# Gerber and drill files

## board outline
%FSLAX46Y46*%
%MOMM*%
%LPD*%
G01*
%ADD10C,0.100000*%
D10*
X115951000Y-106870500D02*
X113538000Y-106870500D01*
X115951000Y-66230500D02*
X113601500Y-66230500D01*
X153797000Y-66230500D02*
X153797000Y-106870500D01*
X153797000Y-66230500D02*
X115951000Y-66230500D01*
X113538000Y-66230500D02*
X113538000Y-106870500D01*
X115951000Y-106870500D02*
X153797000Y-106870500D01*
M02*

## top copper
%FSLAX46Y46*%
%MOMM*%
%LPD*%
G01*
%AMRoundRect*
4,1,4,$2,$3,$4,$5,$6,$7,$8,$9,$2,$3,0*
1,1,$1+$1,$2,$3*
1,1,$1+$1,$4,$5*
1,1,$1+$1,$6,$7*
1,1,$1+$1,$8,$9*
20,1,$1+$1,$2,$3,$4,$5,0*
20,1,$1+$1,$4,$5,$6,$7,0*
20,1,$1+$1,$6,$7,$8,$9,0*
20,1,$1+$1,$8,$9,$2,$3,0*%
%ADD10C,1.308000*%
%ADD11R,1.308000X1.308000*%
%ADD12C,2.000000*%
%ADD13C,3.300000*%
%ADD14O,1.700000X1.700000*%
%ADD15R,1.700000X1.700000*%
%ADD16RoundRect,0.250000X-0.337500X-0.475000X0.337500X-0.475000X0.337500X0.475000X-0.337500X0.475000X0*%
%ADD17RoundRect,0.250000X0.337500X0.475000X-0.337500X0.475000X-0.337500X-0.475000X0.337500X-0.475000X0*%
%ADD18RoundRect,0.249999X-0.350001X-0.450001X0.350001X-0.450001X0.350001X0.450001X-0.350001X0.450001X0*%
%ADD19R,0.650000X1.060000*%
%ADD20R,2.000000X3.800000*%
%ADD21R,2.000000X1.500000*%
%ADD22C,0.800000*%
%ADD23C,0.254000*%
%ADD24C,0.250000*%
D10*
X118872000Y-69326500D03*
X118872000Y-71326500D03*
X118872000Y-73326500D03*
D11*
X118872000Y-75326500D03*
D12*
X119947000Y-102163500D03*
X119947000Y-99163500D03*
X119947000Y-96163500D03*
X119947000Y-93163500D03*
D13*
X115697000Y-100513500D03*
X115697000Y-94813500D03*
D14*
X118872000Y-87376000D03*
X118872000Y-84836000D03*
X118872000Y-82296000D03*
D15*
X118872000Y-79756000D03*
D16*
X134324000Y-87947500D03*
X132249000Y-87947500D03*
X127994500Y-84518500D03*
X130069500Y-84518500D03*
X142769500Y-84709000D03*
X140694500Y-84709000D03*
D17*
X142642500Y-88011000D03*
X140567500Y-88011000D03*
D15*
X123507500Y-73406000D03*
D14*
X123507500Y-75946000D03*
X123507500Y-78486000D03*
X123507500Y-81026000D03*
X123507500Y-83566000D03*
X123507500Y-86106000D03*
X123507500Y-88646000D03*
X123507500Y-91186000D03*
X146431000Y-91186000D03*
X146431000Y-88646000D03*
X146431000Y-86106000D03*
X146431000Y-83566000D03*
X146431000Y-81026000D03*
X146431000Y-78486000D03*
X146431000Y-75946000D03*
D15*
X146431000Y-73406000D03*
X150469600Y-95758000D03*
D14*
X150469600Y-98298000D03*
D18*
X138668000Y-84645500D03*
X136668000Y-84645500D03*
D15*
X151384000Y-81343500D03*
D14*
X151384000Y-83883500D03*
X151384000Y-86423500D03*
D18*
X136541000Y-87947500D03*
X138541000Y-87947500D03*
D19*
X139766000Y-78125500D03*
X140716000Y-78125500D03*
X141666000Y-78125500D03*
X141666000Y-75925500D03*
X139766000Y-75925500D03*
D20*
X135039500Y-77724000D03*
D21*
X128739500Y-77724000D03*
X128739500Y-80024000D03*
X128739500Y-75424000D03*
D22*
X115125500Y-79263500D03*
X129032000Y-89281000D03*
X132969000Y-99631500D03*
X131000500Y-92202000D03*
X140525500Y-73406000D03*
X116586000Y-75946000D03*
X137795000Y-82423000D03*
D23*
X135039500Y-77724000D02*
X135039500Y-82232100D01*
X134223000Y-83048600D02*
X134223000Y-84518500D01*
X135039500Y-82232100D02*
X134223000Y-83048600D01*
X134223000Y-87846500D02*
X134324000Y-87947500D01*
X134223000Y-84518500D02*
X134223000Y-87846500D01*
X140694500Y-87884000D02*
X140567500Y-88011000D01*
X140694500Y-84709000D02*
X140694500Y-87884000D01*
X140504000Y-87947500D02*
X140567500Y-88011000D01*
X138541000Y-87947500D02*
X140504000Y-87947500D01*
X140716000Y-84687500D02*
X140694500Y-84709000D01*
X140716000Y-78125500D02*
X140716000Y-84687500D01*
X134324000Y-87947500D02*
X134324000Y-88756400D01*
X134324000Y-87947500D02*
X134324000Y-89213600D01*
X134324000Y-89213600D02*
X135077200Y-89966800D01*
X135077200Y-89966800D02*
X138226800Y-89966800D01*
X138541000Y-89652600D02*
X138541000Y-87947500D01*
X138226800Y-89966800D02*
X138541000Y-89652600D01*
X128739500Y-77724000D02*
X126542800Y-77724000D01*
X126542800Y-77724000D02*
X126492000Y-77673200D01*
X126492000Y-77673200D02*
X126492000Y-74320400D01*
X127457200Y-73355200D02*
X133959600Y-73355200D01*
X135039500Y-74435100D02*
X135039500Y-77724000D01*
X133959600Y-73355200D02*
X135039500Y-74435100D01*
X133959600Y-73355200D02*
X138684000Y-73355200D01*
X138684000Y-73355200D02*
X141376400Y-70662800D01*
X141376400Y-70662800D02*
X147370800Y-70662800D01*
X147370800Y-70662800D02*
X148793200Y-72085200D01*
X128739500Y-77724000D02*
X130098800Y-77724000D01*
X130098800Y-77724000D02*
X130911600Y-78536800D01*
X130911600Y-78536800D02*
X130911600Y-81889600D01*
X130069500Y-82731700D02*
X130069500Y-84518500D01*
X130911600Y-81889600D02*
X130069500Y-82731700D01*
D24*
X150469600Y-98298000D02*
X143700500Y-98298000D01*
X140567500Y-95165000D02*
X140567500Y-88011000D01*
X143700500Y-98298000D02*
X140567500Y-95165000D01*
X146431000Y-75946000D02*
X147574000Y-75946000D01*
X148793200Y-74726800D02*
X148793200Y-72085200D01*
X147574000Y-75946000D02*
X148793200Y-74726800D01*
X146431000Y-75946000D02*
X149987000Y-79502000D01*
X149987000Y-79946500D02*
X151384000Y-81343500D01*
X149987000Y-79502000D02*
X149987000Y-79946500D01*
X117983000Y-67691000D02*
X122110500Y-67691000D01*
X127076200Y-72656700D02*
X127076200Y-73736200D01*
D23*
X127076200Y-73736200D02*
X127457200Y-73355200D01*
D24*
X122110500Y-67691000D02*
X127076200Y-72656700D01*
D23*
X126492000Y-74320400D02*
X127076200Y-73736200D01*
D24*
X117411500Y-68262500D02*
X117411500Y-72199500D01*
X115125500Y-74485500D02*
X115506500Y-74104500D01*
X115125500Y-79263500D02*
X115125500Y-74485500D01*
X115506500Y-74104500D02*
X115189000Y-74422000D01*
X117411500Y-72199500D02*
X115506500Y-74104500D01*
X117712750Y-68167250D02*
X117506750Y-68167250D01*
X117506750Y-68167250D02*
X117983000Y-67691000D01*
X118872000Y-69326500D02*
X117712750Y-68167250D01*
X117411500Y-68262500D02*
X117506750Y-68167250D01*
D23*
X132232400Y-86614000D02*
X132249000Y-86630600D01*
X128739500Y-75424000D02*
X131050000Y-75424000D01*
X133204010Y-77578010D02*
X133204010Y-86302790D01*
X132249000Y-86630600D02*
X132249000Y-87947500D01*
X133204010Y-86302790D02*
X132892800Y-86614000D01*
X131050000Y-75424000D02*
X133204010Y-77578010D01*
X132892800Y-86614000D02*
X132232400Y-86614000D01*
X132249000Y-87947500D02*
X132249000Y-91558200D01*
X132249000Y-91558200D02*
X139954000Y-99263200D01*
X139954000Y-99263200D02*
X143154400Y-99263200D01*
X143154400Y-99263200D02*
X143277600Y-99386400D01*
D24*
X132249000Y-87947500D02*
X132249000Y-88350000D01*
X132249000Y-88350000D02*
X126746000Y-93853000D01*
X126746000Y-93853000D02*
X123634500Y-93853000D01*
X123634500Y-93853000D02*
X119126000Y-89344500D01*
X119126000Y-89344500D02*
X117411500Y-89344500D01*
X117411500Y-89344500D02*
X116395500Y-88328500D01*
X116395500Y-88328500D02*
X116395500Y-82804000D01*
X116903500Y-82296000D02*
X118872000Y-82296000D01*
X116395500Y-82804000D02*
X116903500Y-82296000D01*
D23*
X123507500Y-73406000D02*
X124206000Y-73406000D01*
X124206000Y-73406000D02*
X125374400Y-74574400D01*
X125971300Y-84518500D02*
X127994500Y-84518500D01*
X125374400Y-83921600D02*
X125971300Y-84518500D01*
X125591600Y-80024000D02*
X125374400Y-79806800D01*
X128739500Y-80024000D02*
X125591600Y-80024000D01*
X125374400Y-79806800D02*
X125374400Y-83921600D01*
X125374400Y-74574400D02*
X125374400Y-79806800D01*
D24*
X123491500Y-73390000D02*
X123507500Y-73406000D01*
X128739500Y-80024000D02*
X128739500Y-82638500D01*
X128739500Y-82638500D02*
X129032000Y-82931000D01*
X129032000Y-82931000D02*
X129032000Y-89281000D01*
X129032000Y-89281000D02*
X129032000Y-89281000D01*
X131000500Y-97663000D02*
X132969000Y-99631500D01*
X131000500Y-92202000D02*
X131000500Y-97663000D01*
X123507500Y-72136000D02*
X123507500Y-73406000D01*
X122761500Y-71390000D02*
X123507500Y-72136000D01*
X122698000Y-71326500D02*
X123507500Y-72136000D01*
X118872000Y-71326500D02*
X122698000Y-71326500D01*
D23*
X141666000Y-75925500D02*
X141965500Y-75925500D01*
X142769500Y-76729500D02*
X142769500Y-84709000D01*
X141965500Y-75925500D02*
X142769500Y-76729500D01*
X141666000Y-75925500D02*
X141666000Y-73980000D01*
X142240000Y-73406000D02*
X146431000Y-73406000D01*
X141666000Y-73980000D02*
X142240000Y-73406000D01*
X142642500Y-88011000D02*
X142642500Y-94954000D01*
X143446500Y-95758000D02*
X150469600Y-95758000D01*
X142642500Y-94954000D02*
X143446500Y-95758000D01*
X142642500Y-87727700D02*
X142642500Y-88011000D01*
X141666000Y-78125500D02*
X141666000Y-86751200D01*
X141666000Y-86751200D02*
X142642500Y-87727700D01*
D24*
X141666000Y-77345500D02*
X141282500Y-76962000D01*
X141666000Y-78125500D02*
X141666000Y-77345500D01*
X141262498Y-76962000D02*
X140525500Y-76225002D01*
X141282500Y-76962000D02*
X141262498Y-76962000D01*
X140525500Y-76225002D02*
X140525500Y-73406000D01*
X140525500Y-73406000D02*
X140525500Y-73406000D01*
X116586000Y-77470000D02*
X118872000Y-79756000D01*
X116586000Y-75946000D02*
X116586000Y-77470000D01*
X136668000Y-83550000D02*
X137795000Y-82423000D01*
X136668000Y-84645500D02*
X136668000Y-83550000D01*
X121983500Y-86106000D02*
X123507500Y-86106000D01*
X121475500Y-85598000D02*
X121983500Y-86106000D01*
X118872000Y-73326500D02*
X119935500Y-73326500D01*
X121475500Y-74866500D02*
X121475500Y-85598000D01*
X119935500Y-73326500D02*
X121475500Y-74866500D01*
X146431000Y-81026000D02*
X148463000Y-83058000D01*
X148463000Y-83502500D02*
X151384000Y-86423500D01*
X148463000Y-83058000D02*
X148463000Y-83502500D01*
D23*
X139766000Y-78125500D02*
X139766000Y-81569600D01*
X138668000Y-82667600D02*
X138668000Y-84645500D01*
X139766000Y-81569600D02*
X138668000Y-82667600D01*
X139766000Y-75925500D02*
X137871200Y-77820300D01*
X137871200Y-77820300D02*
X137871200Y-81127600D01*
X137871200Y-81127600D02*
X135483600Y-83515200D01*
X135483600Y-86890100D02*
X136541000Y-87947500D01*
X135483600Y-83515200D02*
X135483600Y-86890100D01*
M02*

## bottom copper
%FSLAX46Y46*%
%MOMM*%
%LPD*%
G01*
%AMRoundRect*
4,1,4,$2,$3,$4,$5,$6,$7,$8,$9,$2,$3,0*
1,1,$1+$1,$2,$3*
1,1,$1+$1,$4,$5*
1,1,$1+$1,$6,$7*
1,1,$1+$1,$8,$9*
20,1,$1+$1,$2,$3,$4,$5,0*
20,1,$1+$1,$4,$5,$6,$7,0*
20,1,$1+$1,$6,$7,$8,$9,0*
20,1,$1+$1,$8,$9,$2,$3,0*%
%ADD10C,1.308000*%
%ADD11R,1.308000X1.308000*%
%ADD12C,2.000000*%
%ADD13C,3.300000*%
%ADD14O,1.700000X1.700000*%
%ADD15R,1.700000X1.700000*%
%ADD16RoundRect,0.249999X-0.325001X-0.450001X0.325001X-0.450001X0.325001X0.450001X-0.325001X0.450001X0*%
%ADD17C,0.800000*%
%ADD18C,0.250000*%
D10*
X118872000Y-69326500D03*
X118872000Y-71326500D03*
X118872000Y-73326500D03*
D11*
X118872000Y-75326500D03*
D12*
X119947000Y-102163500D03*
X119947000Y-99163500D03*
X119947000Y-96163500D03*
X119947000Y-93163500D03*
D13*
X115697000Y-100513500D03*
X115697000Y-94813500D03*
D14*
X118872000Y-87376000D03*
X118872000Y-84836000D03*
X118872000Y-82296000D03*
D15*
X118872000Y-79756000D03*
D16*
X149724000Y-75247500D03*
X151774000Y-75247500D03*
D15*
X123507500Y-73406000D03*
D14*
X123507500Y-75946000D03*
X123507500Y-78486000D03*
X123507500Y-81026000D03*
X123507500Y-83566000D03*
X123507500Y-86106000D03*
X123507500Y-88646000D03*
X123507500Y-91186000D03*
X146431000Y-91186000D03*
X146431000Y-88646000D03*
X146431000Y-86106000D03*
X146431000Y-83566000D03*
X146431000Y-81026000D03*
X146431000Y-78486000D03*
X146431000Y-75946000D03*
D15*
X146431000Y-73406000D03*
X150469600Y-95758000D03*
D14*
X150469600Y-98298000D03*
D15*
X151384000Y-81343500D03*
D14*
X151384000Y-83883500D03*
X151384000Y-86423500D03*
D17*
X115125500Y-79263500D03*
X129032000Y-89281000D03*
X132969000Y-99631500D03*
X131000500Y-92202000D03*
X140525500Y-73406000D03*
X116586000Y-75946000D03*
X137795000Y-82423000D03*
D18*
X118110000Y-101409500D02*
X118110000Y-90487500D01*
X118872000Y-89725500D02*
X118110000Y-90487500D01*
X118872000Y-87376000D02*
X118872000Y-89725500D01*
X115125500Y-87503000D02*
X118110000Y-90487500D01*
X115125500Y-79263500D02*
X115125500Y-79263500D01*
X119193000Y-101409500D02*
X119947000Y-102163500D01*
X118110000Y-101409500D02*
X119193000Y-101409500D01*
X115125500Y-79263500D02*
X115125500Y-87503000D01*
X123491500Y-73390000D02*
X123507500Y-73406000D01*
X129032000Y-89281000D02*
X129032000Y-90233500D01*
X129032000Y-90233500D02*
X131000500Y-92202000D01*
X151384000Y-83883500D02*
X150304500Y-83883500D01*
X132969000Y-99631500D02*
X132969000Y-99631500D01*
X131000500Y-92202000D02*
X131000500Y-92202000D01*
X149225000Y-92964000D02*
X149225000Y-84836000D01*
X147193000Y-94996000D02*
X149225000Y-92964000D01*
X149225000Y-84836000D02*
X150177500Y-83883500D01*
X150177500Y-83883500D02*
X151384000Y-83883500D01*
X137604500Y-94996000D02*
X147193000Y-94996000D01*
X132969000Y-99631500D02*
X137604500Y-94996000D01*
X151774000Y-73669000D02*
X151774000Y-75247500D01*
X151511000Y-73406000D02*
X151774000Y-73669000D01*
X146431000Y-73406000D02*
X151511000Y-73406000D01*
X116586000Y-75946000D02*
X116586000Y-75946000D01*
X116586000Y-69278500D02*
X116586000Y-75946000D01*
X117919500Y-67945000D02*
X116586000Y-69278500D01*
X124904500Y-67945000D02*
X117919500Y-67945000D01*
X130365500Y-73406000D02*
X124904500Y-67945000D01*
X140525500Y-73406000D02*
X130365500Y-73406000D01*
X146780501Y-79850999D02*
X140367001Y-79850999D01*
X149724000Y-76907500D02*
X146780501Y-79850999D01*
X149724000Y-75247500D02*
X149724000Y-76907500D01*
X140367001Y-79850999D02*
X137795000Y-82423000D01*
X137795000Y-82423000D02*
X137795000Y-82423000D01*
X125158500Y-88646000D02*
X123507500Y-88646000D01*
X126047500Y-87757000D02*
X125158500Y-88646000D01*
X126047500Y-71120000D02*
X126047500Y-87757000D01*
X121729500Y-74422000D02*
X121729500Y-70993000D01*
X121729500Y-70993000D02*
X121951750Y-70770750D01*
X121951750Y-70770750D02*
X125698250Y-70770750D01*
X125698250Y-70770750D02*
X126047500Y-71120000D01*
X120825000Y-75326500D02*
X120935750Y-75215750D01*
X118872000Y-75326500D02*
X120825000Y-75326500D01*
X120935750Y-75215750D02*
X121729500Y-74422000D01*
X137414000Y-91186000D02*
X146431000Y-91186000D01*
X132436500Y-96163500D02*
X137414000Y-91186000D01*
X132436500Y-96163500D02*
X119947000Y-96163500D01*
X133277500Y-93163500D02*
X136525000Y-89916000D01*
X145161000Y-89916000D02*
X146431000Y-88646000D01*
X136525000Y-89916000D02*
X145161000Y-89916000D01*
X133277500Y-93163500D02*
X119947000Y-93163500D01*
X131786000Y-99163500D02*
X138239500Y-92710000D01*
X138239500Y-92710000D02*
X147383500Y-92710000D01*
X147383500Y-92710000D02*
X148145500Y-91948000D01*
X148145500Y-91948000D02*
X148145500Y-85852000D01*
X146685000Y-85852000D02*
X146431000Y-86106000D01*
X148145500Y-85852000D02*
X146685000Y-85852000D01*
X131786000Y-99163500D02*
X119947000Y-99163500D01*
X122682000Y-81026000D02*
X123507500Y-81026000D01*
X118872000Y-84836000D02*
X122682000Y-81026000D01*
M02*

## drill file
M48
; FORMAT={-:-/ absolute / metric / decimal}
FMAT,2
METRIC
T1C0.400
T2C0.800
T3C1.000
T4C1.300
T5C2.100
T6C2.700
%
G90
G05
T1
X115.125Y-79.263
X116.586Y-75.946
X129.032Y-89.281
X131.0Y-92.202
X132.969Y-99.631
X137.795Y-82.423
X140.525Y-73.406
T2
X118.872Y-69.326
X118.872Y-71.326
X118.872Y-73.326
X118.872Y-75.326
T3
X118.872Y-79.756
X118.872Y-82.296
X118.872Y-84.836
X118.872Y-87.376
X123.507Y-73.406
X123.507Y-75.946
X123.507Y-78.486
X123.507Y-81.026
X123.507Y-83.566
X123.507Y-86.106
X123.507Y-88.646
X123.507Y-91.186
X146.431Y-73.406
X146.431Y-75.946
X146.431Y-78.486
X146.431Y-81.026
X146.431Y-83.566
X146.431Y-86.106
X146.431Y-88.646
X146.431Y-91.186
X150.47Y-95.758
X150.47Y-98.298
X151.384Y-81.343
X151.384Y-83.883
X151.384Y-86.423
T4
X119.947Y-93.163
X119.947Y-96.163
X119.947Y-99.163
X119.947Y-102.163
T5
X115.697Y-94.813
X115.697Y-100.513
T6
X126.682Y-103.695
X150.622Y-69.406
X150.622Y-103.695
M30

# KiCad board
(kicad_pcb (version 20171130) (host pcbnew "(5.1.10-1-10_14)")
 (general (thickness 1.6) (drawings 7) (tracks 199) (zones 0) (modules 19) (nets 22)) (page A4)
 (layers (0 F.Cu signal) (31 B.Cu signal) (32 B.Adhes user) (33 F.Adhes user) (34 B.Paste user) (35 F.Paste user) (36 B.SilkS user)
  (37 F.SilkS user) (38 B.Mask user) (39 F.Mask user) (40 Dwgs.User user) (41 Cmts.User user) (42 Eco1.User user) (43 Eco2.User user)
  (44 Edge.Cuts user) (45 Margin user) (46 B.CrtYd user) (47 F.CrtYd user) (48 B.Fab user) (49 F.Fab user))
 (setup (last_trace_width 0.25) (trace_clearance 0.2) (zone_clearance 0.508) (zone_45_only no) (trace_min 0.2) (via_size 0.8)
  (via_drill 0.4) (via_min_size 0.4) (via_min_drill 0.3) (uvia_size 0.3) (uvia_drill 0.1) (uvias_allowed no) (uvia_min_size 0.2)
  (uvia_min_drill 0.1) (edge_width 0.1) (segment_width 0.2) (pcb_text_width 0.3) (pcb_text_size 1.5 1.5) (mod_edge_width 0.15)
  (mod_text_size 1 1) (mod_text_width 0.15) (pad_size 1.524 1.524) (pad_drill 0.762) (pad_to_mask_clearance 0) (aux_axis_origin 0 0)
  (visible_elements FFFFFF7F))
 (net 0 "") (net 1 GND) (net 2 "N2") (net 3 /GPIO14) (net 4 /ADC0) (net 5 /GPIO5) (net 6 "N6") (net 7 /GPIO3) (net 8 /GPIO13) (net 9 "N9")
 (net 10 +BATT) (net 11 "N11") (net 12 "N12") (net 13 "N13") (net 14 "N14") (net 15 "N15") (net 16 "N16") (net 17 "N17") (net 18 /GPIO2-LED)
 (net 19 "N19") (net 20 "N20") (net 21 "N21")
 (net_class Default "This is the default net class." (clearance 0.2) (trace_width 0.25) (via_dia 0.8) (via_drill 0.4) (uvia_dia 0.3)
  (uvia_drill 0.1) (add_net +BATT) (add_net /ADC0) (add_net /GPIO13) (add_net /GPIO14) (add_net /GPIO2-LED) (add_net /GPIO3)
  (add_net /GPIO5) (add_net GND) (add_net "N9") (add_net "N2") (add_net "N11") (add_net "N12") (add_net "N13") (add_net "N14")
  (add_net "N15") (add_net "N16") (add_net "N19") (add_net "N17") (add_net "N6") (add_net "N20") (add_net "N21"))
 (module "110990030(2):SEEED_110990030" (layer F.Cu) (at 118.872 72.3265 90)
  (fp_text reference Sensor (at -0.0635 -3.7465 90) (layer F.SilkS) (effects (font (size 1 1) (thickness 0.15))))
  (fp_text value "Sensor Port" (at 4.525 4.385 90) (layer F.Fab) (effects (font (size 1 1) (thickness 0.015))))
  (pad 4 thru_hole circle (at 3 0 90) (size 1.308 1.308) (drill 0.8) (layers *.Cu *.Mask) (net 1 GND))
  (pad 3 thru_hole circle (at 1 0 90) (size 1.308 1.308) (drill 0.8) (layers *.Cu *.Mask) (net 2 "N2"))
  (pad 2 thru_hole circle (at -1 0 90) (size 1.308 1.308) (drill 0.8) (layers *.Cu *.Mask) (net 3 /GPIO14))
  (pad 1 thru_hole rect (at -3 0 90) (size 1.308 1.308) (drill 0.8) (layers *.Cu *.Mask) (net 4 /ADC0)))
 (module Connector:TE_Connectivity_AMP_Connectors (layer F.Cu) (at 115.697 95.3135 270)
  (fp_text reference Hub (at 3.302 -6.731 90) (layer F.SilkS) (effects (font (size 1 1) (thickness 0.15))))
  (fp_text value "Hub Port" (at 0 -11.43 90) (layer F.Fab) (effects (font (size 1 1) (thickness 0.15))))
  (pad 4 thru_hole circle (at 6.85 -4.25 270) (size 2 2) (drill 1.3) (layers *.Cu *.Mask) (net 1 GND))
  (pad 3 thru_hole circle (at 3.85 -4.25 270) (size 2 2) (drill 1.3) (layers *.Cu *.Mask) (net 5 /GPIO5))
  (pad 2 thru_hole circle (at 0.85 -4.25 270) (size 2 2) (drill 1.3) (layers *.Cu *.Mask) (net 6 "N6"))
  (pad 1 thru_hole circle (at -2.15 -4.25 270) (size 2 2) (drill 1.3) (layers *.Cu *.Mask) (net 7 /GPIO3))
  (pad 6 thru_hole circle (at 5.2 0 270) (size 3.3 3.3) (drill 2.1) (layers *.Cu *.Mask))
  (pad 5 thru_hole circle (at -0.5 0 270) (size 3.3 3.3) (drill 2.1) (layers *.Cu *.Mask)))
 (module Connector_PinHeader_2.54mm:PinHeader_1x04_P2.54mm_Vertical (layer F.Cu) (at 118.872 79.756)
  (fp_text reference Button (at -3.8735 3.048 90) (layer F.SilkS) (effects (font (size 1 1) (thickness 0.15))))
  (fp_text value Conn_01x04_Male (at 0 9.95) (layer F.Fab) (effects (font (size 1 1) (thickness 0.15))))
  (pad 4 thru_hole oval (at 0 7.62) (size 1.7 1.7) (drill 1) (layers *.Cu *.Mask) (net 1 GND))
  (pad 3 thru_hole oval (at 0 5.08) (size 1.7 1.7) (drill 1) (layers *.Cu *.Mask) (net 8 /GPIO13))
  (pad 2 thru_hole oval (at 0 2.54) (size 1.7 1.7) (drill 1) (layers *.Cu *.Mask) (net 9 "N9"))
  (pad 1 thru_hole rect (at 0 0) (size 1.7 1.7) (drill 1) (layers *.Cu *.Mask) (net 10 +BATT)))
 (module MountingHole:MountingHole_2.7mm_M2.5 (layer F.Cu) (at 126.6825 103.6955)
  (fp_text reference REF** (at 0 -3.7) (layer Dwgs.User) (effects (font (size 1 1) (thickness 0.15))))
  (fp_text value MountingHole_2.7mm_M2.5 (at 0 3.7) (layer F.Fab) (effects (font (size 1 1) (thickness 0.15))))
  (pad 1 np_thru_hole circle (at 0 0) (size 2.7 2.7) (drill 2.7) (layers *.Cu *.Mask)))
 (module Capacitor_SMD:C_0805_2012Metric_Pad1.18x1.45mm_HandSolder (layer F.Cu) (at 133.2865 87.9475)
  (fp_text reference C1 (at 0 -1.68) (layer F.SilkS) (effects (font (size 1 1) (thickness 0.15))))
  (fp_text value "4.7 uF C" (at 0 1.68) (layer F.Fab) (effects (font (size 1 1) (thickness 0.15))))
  (pad 2 smd roundrect (at 1.0375 0) (size 1.175 1.45) (layers F.Cu F.Paste F.Mask) (roundrect_rratio 0.2127659574468085) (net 1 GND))
  (pad 1 smd roundrect (at -1.0375 0) (size 1.175 1.45) (layers F.Cu F.Paste F.Mask) (roundrect_rratio 0.2127659574468085) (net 9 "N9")))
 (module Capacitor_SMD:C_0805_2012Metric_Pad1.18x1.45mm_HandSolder (layer F.Cu) (at 129.032 84.5185)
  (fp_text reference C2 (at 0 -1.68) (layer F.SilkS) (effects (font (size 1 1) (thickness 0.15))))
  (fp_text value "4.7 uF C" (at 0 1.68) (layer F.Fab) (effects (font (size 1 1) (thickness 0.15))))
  (pad 1 smd roundrect (at -1.0375 0) (size 1.175 1.45) (layers F.Cu F.Paste F.Mask) (roundrect_rratio 0.2127659574468085) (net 2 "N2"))
  (pad 2 smd roundrect (at 1.0375 0) (size 1.175 1.45) (layers F.Cu F.Paste F.Mask) (roundrect_rratio 0.2127659574468085) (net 1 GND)))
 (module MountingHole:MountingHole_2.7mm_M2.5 (layer F.Cu) (at 150.622 103.6955)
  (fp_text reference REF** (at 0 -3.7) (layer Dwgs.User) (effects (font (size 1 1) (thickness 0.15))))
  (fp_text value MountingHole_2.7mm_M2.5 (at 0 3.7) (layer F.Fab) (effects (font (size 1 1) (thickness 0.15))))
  (pad 1 np_thru_hole circle (at 0 0) (size 2.7 2.7) (drill 2.7) (layers *.Cu *.Mask)))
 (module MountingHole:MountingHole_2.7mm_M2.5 (layer F.Cu) (at 150.622 69.4055)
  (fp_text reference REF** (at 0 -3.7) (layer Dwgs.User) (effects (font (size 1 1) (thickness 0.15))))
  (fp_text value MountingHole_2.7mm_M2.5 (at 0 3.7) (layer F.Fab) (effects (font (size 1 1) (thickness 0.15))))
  (pad 1 np_thru_hole circle (at 0 0) (size 2.7 2.7) (drill 2.7) (layers *.Cu *.Mask)))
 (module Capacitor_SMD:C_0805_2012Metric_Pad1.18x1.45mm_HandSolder (layer F.Cu) (at 141.732 84.709)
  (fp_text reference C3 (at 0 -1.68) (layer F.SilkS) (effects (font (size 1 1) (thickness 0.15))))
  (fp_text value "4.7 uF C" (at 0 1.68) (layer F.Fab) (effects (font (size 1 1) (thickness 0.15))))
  (pad 2 smd roundrect (at 1.0375 0) (size 1.175 1.45) (layers F.Cu F.Paste F.Mask) (roundrect_rratio 0.2127659574468085) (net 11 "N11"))
  (pad 1 smd roundrect (at -1.0375 0) (size 1.175 1.45) (layers F.Cu F.Paste F.Mask) (roundrect_rratio 0.2127659574468085) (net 1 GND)))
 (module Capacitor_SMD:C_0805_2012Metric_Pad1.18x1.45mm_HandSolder (layer F.Cu) (at 141.605 88.011 180)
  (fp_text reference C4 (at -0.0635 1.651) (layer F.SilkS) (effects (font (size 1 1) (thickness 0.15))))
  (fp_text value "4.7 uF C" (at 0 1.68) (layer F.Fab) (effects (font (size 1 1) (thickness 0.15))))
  (pad 1 smd roundrect (at -1.0375 0 180) (size 1.175 1.45) (layers F.Cu F.Paste F.Mask) (roundrect_rratio 0.2127659574468085)
   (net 10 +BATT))
  (pad 2 smd roundrect (at 1.0375 0 180) (size 1.175 1.45) (layers F.Cu F.Paste F.Mask) (roundrect_rratio 0.2127659574468085) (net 1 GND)))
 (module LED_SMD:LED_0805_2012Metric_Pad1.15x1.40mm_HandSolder (layer B.Cu) (at 150.749 75.2475)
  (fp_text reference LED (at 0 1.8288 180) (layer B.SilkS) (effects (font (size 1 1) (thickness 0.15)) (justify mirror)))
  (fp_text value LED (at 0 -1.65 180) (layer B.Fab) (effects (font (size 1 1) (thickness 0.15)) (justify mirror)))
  (pad 1 smd roundrect (at -1.025 0) (size 1.15 1.4) (layers B.Cu B.Paste B.Mask) (roundrect_rratio 0.2173904347826087) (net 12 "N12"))
  (pad 2 smd roundrect (at 1.025 0) (size 1.15 1.4) (layers B.Cu B.Paste B.Mask) (roundrect_rratio 0.2173904347826087) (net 11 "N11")))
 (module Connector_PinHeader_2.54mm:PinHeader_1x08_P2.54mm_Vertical (layer B.Cu) (at 123.5075 73.406 180)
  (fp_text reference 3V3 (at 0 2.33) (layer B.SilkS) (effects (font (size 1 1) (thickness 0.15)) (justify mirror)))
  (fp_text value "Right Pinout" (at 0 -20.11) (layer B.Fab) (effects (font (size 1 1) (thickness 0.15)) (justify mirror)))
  (pad 1 thru_hole rect (at 0 0 180) (size 1.7 1.7) (drill 1) (layers *.Cu *.Mask) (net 2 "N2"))
  (pad 2 thru_hole oval (at 0 -2.54 180) (size 1.7 1.7) (drill 1) (layers *.Cu *.Mask) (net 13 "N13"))
  (pad 3 thru_hole oval (at 0 -5.08 180) (size 1.7 1.7) (drill 1) (layers *.Cu *.Mask) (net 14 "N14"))
  (pad 4 thru_hole oval (at 0 -7.62 180) (size 1.7 1.7) (drill 1) (layers *.Cu *.Mask) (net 8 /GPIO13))
  (pad 5 thru_hole oval (at 0 -10.16 180) (size 1.7 1.7) (drill 1) (layers *.Cu *.Mask) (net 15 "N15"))
  (pad 6 thru_hole oval (at 0 -12.7 180) (size 1.7 1.7) (drill 1) (layers *.Cu *.Mask) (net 3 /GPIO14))
  (pad 7 thru_hole oval (at 0 -15.24 180) (size 1.7 1.7) (drill 1) (layers *.Cu *.Mask) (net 4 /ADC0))
  (pad 8 thru_hole oval (at 0 -17.78 180) (size 1.7 1.7) (drill 1) (layers *.Cu *.Mask) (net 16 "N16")))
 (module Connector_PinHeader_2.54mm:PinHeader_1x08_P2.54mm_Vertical (layer B.Cu) (at 146.431 73.406 180)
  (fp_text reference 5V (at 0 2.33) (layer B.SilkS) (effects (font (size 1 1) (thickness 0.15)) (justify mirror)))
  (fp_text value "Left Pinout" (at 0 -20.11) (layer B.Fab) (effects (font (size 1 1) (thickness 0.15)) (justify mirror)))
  (pad 8 thru_hole oval (at 0 -17.78 180) (size 1.7 1.7) (drill 1) (layers *.Cu *.Mask) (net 6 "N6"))
  (pad 7 thru_hole oval (at 0 -15.24 180) (size 1.7 1.7) (drill 1) (layers *.Cu *.Mask) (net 7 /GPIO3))
  (pad 6 thru_hole oval (at 0 -12.7 180) (size 1.7 1.7) (drill 1) (layers *.Cu *.Mask) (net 5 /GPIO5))
  (pad 5 thru_hole oval (at 0 -10.16 180) (size 1.7 1.7) (drill 1) (layers *.Cu *.Mask) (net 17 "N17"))
  (pad 4 thru_hole oval (at 0 -7.62 180) (size 1.7 1.7) (drill 1) (layers *.Cu *.Mask) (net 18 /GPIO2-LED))
  (pad 3 thru_hole oval (at 0 -5.08 180) (size 1.7 1.7) (drill 1) (layers *.Cu *.Mask) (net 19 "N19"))
  (pad 2 thru_hole oval (at 0 -2.54 180) (size 1.7 1.7) (drill 1) (layers *.Cu *.Mask) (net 1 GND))
  (pad 1 thru_hole rect (at 0 0 180) (size 1.7 1.7) (drill 1) (layers *.Cu *.Mask) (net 11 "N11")))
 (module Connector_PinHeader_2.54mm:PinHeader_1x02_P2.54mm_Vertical (layer F.Cu) (at 150.4696 95.758)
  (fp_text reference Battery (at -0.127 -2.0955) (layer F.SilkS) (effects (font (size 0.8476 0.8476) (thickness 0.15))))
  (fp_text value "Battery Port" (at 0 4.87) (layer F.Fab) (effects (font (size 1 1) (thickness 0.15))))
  (pad 1 thru_hole rect (at 0 0) (size 1.7 1.7) (drill 1) (layers *.Cu *.Mask) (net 10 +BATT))
  (pad 2 thru_hole oval (at 0 2.54) (size 1.7 1.7) (drill 1) (layers *.Cu *.Mask) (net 1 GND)))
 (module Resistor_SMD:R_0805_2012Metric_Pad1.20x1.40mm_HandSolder (layer F.Cu) (at 137.668 84.6455)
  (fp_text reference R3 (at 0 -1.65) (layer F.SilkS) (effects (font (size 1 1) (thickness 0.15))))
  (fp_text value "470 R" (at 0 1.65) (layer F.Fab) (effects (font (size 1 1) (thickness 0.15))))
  (pad 2 smd roundrect (at 1 0) (size 1.2 1.4) (layers F.Cu F.Paste F.Mask) (roundrect_rratio 0.2083325) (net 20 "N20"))
  (pad 1 smd roundrect (at -1 0) (size 1.2 1.4) (layers F.Cu F.Paste F.Mask) (roundrect_rratio 0.2083325) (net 12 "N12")))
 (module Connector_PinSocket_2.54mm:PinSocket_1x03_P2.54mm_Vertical (layer F.Cu) (at 151.384 81.3435)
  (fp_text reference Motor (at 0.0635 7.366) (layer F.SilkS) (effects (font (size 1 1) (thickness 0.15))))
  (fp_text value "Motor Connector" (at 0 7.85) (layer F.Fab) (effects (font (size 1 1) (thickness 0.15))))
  (pad 1 thru_hole rect (at 0 0) (size 1.7 1.7) (drill 1) (layers *.Cu *.Mask) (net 1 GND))
  (pad 2 thru_hole oval (at 0 2.54) (size 1.7 1.7) (drill 1) (layers *.Cu *.Mask) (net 2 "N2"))
  (pad 3 thru_hole oval (at 0 5.08) (size 1.7 1.7) (drill 1) (layers *.Cu *.Mask) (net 18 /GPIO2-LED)))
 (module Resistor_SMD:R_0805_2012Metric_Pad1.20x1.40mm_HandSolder (layer F.Cu) (at 137.541 87.9475)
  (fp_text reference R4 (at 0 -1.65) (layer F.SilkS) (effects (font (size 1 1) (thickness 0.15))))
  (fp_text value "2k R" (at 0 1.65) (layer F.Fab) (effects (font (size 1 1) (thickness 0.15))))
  (pad 1 smd roundrect (at -1 0) (size 1.2 1.4) (layers F.Cu F.Paste F.Mask) (roundrect_rratio 0.2083325) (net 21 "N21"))
  (pad 2 smd roundrect (at 1 0) (size 1.2 1.4) (layers F.Cu F.Paste F.Mask) (roundrect_rratio 0.2083325) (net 1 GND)))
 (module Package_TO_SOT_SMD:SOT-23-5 (layer F.Cu) (at 140.716 77.0255 90)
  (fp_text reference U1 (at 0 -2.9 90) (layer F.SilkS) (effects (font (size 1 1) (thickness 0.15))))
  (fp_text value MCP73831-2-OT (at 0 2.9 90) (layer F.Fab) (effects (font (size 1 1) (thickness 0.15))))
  (pad 1 smd rect (at -1.1 -0.95 90) (size 1.06 0.65) (layers F.Cu F.Paste F.Mask) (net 20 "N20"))
  (pad 2 smd rect (at -1.1 0 90) (size 1.06 0.65) (layers F.Cu F.Paste F.Mask) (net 1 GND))
  (pad 3 smd rect (at -1.1 0.95 90) (size 1.06 0.65) (layers F.Cu F.Paste F.Mask) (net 10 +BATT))
  (pad 4 smd rect (at 1.1 0.95 90) (size 1.06 0.65) (layers F.Cu F.Paste F.Mask) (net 11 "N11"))
  (pad 5 smd rect (at 1.1 -0.95 90) (size 1.06 0.65) (layers F.Cu F.Paste F.Mask) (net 21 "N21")))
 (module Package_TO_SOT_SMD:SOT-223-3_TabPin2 (layer F.Cu) (at 131.8895 77.724)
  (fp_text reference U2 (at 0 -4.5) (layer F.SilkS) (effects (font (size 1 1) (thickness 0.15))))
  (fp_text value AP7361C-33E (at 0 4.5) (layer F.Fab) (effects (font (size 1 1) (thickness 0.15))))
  (pad 2 smd rect (at 3.15 0) (size 2 3.8) (layers F.Cu F.Paste F.Mask) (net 1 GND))
  (pad 2 smd rect (at -3.15 0) (size 2 1.5) (layers F.Cu F.Paste F.Mask) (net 1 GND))
  (pad 3 smd rect (at -3.15 2.3) (size 2 1.5) (layers F.Cu F.Paste F.Mask) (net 2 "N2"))
  (pad 1 smd rect (at -3.15 -2.3) (size 2 1.5) (layers F.Cu F.Paste F.Mask) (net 9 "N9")))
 (gr_line (start 115.951 106.8705) (end 113.538 106.8705) (layer Edge.Cuts) (width 0.1))
 (gr_line (start 115.951 66.2305) (end 113.6015 66.2305) (layer Edge.Cuts) (width 0.1))
 (gr_line (start 153.797 66.2305) (end 153.797 106.8705) (layer Edge.Cuts) (width 0.1))
 (gr_line (start 153.797 66.2305) (end 115.951 66.2305) (layer Edge.Cuts) (width 0.1))
 (gr_line (start 113.538 66.2305) (end 113.538 106.8705) (layer Edge.Cuts) (width 0.1))
 (gr_line (start 115.951 106.8705) (end 153.797 106.8705) (layer Edge.Cuts) (width 0.1))
 (segment (start 135.0395 77.724) (end 135.0395 82.2321) (width 0.254) (layer F.Cu) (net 1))
 (segment (start 134.223 83.0486) (end 134.223 84.5185) (width 0.254) (layer F.Cu) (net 1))
 (segment (start 135.0395 82.2321) (end 134.223 83.0486) (width 0.254) (layer F.Cu) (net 1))
 (segment (start 134.223 87.8465) (end 134.324 87.9475) (width 0.254) (layer F.Cu) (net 1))
 (segment (start 134.223 84.5185) (end 134.223 87.8465) (width 0.254) (layer F.Cu) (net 1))
 (segment (start 140.6945 87.884) (end 140.5675 88.011) (width 0.254) (layer F.Cu) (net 1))
 (segment (start 140.6945 84.709) (end 140.6945 87.884) (width 0.254) (layer F.Cu) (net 1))
 (segment (start 140.504 87.9475) (end 140.5675 88.011) (width 0.254) (layer F.Cu) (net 1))
 (segment (start 138.541 87.9475) (end 140.504 87.9475) (width 0.254) (layer F.Cu) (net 1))
 (segment (start 140.716 84.6875) (end 140.6945 84.709) (width 0.254) (layer F.Cu) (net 1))
 (segment (start 140.716 78.1255) (end 140.716 84.6875) (width 0.254) (layer F.Cu) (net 1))
 (segment (start 134.324 87.9475) (end 134.324 88.7564) (width 0.254) (layer F.Cu) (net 1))
 (segment (start 134.324 87.9475) (end 134.324 89.2136) (width 0.254) (layer F.Cu) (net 1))
 (segment (start 134.324 89.2136) (end 135.0772 89.9668) (width 0.254) (layer F.Cu) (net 1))
 (segment (start 135.0772 89.9668) (end 138.2268 89.9668) (width 0.254) (layer F.Cu) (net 1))
 (segment (start 138.541 89.6526) (end 138.541 87.9475) (width 0.254) (layer F.Cu) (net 1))
 (segment (start 138.2268 89.9668) (end 138.541 89.6526) (width 0.254) (layer F.Cu) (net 1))
 (segment (start 128.7395 77.724) (end 126.5428 77.724) (width 0.254) (layer F.Cu) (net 1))
 (segment (start 126.5428 77.724) (end 126.492 77.6732) (width 0.254) (layer F.Cu) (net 1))
 (segment (start 126.492 77.6732) (end 126.492 74.3204) (width 0.254) (layer F.Cu) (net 1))
 (segment (start 127.4572 73.3552) (end 133.9596 73.3552) (width 0.254) (layer F.Cu) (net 1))
 (segment (start 135.0395 74.4351) (end 135.0395 77.724) (width 0.254) (layer F.Cu) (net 1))
 (segment (start 133.9596 73.3552) (end 135.0395 74.4351) (width 0.254) (layer F.Cu) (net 1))
 (segment (start 133.9596 73.3552) (end 138.684 73.3552) (width 0.254) (layer F.Cu) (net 1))
 (segment (start 138.684 73.3552) (end 141.3764 70.6628) (width 0.254) (layer F.Cu) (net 1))
 (segment (start 141.3764 70.6628) (end 147.3708 70.6628) (width 0.254) (layer F.Cu) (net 1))
 (segment (start 147.3708 70.6628) (end 148.7932 72.0852) (width 0.254) (layer F.Cu) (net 1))
 (segment (start 128.7395 77.724) (end 130.0988 77.724) (width 0.254) (layer F.Cu) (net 1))
 (segment (start 130.0988 77.724) (end 130.9116 78.5368) (width 0.254) (layer F.Cu) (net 1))
 (segment (start 130.9116 78.5368) (end 130.9116 81.8896) (width 0.254) (layer F.Cu) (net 1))
 (segment (start 130.0695 82.7317) (end 130.0695 84.5185) (width 0.254) (layer F.Cu) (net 1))
 (segment (start 130.9116 81.8896) (end 130.0695 82.7317) (width 0.254) (layer F.Cu) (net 1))
 (segment (start 150.4696 98.298) (end 143.7005 98.298) (width 0.25) (layer F.Cu) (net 1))
 (segment (start 140.5675 95.165) (end 140.5675 88.011) (width 0.25) (layer F.Cu) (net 1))
 (segment (start 143.7005 98.298) (end 140.5675 95.165) (width 0.25) (layer F.Cu) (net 1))
 (segment (start 118.11 101.4095) (end 118.11 90.4875) (width 0.25) (layer B.Cu) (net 1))
 (segment (start 118.872 89.7255) (end 118.11 90.4875) (width 0.25) (layer B.Cu) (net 1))
 (segment (start 118.872 87.376) (end 118.872 89.7255) (width 0.25) (layer B.Cu) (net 1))
 (segment (start 146.431 75.946) (end 147.574 75.946) (width 0.25) (layer F.Cu) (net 1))
 (segment (start 148.7932 74.7268) (end 148.7932 72.0852) (width 0.25) (layer F.Cu) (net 1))
 (segment (start 147.574 75.946) (end 148.7932 74.7268) (width 0.25) (layer F.Cu) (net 1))
 (segment (start 146.431 75.946) (end 149.987 79.502) (width 0.25) (layer F.Cu) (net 1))
 (segment (start 149.987 79.9465) (end 151.384 81.3435) (width 0.25) (layer F.Cu) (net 1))
 (segment (start 149.987 79.502) (end 149.987 79.9465) (width 0.25) (layer F.Cu) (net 1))
 (segment (start 115.1255 87.503) (end 118.11 90.4875) (width 0.25) (layer B.Cu) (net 1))
 (segment (start 115.1255 79.2635) (end 115.1255 79.2635) (width 0.25) (layer B.Cu) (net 1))
 (segment (start 117.983 67.691) (end 122.1105 67.691) (width 0.25) (layer F.Cu) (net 1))
 (segment (start 127.0762 72.6567) (end 127.0762 73.7362) (width 0.25) (layer F.Cu) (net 1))
 (segment (start 127.0762 73.7362) (end 127.4572 73.3552) (width 0.254) (layer F.Cu) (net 1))
 (segment (start 122.1105 67.691) (end 127.0762 72.6567) (width 0.25) (layer F.Cu) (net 1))
 (segment (start 126.492 74.3204) (end 127.0762 73.7362) (width 0.254) (layer F.Cu) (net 1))
 (segment (start 119.193 101.4095) (end 119.947 102.1635) (width 0.25) (layer B.Cu) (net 1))
 (segment (start 118.11 101.4095) (end 119.193 101.4095) (width 0.25) (layer B.Cu) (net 1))
 (segment (start 117.4115 68.2625) (end 117.4115 72.1995) (width 0.25) (layer F.Cu) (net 1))
 (segment (start 115.1255 79.2635) (end 115.1255 87.503) (width 0.25) (layer B.Cu) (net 1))
 (via (at 115.1255 79.2635) (size 0.8) (drill 0.4) (layers F.Cu B.Cu) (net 1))
 (segment (start 115.1255 74.4855) (end 115.5065 74.1045) (width 0.25) (layer F.Cu) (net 1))
 (segment (start 115.1255 79.2635) (end 115.1255 74.4855) (width 0.25) (layer F.Cu) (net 1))
 (segment (start 115.5065 74.1045) (end 115.189 74.422) (width 0.25) (layer F.Cu) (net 1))
 (segment (start 117.4115 72.1995) (end 115.5065 74.1045) (width 0.25) (layer F.Cu) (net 1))
 (segment (start 117.71275 68.16725) (end 117.50675 68.16725) (width 0.25) (layer F.Cu) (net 1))
 (segment (start 117.50675 68.16725) (end 117.983 67.691) (width 0.25) (layer F.Cu) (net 1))
 (segment (start 118.872 69.3265) (end 117.71275 68.16725) (width 0.25) (layer F.Cu) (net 1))
 (segment (start 117.4115 68.2625) (end 117.50675 68.16725) (width 0.25) (layer F.Cu) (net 1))
 (segment (start 132.2324 86.614) (end 132.249 86.6306) (width 0.254) (layer F.Cu) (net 9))
 (segment (start 128.7395 75.424) (end 131.05 75.424) (width 0.254) (layer F.Cu) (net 9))
 (segment (start 133.20401 77.57801) (end 133.20401 86.30279) (width 0.254) (layer F.Cu) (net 9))
 (segment (start 132.249 86.6306) (end 132.249 87.9475) (width 0.254) (layer F.Cu) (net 9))
 (segment (start 133.20401 86.30279) (end 132.8928 86.614) (width 0.254) (layer F.Cu) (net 9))
 (segment (start 131.05 75.424) (end 133.20401 77.57801) (width 0.254) (layer F.Cu) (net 9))
 (segment (start 132.8928 86.614) (end 132.2324 86.614) (width 0.254) (layer F.Cu) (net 9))
 (segment (start 132.249 87.9475) (end 132.249 91.5582) (width 0.254) (layer F.Cu) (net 9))
 (segment (start 132.249 91.5582) (end 139.954 99.2632) (width 0.254) (layer F.Cu) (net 9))
 (segment (start 139.954 99.2632) (end 143.1544 99.2632) (width 0.254) (layer F.Cu) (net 9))
 (segment (start 143.1544 99.2632) (end 143.2776 99.3864) (width 0.254) (layer F.Cu) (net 9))
 (segment (start 132.249 87.9475) (end 132.249 88.35) (width 0.25) (layer F.Cu) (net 9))
 (segment (start 132.249 88.35) (end 126.746 93.853) (width 0.25) (layer F.Cu) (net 9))
 (segment (start 126.746 93.853) (end 123.6345 93.853) (width 0.25) (layer F.Cu) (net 9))
 (segment (start 123.6345 93.853) (end 119.126 89.3445) (width 0.25) (layer F.Cu) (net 9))
 (segment (start 119.126 89.3445) (end 117.4115 89.3445) (width 0.25) (layer F.Cu) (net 9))
 (segment (start 117.4115 89.3445) (end 116.3955 88.3285) (width 0.25) (layer F.Cu) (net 9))
 (segment (start 116.3955 88.3285) (end 116.3955 82.804) (width 0.25) (layer F.Cu) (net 9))
 (segment (start 116.9035 82.296) (end 118.872 82.296) (width 0.25) (layer F.Cu) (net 9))
 (segment (start 116.3955 82.804) (end 116.9035 82.296) (width 0.25) (layer F.Cu) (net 9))
 (segment (start 123.5075 73.406) (end 124.206 73.406) (width 0.254) (layer F.Cu) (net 2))
 (segment (start 124.206 73.406) (end 125.3744 74.5744) (width 0.254) (layer F.Cu) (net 2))
 (segment (start 125.9713 84.5185) (end 127.9945 84.5185) (width 0.254) (layer F.Cu) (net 2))
 (segment (start 125.3744 83.9216) (end 125.9713 84.5185) (width 0.254) (layer F.Cu) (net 2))
 (segment (start 125.5916 80.024) (end 125.3744 79.8068) (width 0.254) (layer F.Cu) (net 2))
 (segment (start 128.7395 80.024) (end 125.5916 80.024) (width 0.254) (layer F.Cu) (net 2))
 (segment (start 125.3744 79.8068) (end 125.3744 83.9216) (width 0.254) (layer F.Cu) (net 2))
 (segment (start 125.3744 74.5744) (end 125.3744 79.8068) (width 0.254) (layer F.Cu) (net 2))
 (segment (start 123.4915 73.39) (end 123.5075 73.406) (width 0.25) (layer F.Cu) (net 2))
 (segment (start 123.4915 73.39) (end 123.5075 73.406) (width 0.25) (layer B.Cu) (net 2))
 (segment (start 128.7395 80.024) (end 128.7395 82.6385) (width 0.25) (layer F.Cu) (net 2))
 (segment (start 128.7395 82.6385) (end 129.032 82.931) (width 0.25) (layer F.Cu) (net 2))
 (segment (start 129.032 82.931) (end 129.032 89.281) (width 0.25) (layer F.Cu) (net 2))
 (segment (start 129.032 89.281) (end 129.032 89.281) (width 0.25) (layer F.Cu) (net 2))
 (via (at 129.032 89.281) (size 0.8) (drill 0.4) (layers F.Cu B.Cu) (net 2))
 (segment (start 129.032 89.281) (end 129.032 90.2335) (width 0.25) (layer B.Cu) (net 2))
 (segment (start 129.032 90.2335) (end 131.0005 92.202) (width 0.25) (layer B.Cu) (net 2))
 (segment (start 151.384 83.8835) (end 150.3045 83.8835) (width 0.25) (layer B.Cu) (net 2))
 (segment (start 132.969 99.6315) (end 132.969 99.6315) (width 0.25) (layer B.Cu) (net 2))
 (via (at 132.969 99.6315) (size 0.8) (drill 0.4) (layers F.Cu B.Cu) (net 2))
 (segment (start 131.0005 92.202) (end 131.0005 92.202) (width 0.25) (layer B.Cu) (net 2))
 (via (at 131.0005 92.202) (size 0.8) (drill 0.4) (layers F.Cu B.Cu) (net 2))
 (segment (start 131.0005 97.663) (end 132.969 99.6315) (width 0.25) (layer F.Cu) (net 2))
 (segment (start 131.0005 92.202) (end 131.0005 97.663) (width 0.25) (layer F.Cu) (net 2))
 (segment (start 123.5075 72.136) (end 123.5075 73.406) (width 0.25) (layer F.Cu) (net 2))
 (segment (start 122.7615 71.39) (end 123.5075 72.136) (width 0.25) (layer F.Cu) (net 2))
 (segment (start 122.698 71.3265) (end 123.5075 72.136) (width 0.25) (layer F.Cu) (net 2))
 (segment (start 118.872 71.3265) (end 122.698 71.3265) (width 0.25) (layer F.Cu) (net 2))
 (segment (start 149.225 92.964) (end 149.225 84.836) (width 0.25) (layer B.Cu) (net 2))
 (segment (start 147.193 94.996) (end 149.225 92.964) (width 0.25) (layer B.Cu) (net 2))
 (segment (start 149.225 84.836) (end 150.1775 83.8835) (width 0.25) (layer B.Cu) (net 2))
 (segment (start 150.1775 83.8835) (end 151.384 83.8835) (width 0.25) (layer B.Cu) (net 2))
 (segment (start 137.6045 94.996) (end 147.193 94.996) (width 0.25) (layer B.Cu) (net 2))
 (segment (start 132.969 99.6315) (end 137.6045 94.996) (width 0.25) (layer B.Cu) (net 2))
 (segment (start 141.666 75.9255) (end 141.9655 75.9255) (width 0.254) (layer F.Cu) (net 11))
 (segment (start 142.7695 76.7295) (end 142.7695 84.709) (width 0.254) (layer F.Cu) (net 11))
 (segment (start 141.9655 75.9255) (end 142.7695 76.7295) (width 0.254) (layer F.Cu) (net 11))
 (segment (start 141.666 75.9255) (end 141.666 73.98) (width 0.254) (layer F.Cu) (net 11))
 (segment (start 142.24 73.406) (end 146.431 73.406) (width 0.254) (layer F.Cu) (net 11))
 (segment (start 141.666 73.98) (end 142.24 73.406) (width 0.254) (layer F.Cu) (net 11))
 (segment (start 151.774 73.669) (end 151.774 75.2475) (width 0.25) (layer B.Cu) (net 11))
 (segment (start 151.511 73.406) (end 151.774 73.669) (width 0.25) (layer B.Cu) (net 11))
 (segment (start 146.431 73.406) (end 151.511 73.406) (width 0.25) (layer B.Cu) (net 11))
 (segment (start 142.6425 88.011) (end 142.6425 94.954) (width 0.254) (layer F.Cu) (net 10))
 (segment (start 143.4465 95.758) (end 150.4696 95.758) (width 0.254) (layer F.Cu) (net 10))
 (segment (start 142.6425 94.954) (end 143.4465 95.758) (width 0.254) (layer F.Cu) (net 10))
 (segment (start 142.6425 87.7277) (end 142.6425 88.011) (width 0.254) (layer F.Cu) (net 10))
 (segment (start 141.666 78.1255) (end 141.666 86.7512) (width 0.254) (layer F.Cu) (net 10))
 (segment (start 141.666 86.7512) (end 142.6425 87.7277) (width 0.254) (layer F.Cu) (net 10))
 (segment (start 141.666 77.3455) (end 141.2825 76.962) (width 0.25) (layer F.Cu) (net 10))
 (segment (start 141.666 78.1255) (end 141.666 77.3455) (width 0.25) (layer F.Cu) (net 10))
 (segment (start 141.262498 76.962) (end 140.5255 76.225002) (width 0.25) (layer F.Cu) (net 10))
 (segment (start 141.2825 76.962) (end 141.262498 76.962) (width 0.25) (layer F.Cu) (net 10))
 (segment (start 140.5255 76.225002) (end 140.5255 73.406) (width 0.25) (layer F.Cu) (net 10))
 (segment (start 140.5255 73.406) (end 140.5255 73.406) (width 0.25) (layer F.Cu) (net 10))
 (via (at 140.5255 73.406) (size 0.8) (drill 0.4) (layers F.Cu B.Cu) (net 10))
 (segment (start 116.586 75.946) (end 116.586 75.946) (width 0.25) (layer B.Cu) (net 10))
 (via (at 116.586 75.946) (size 0.8) (drill 0.4) (layers F.Cu B.Cu) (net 10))
 (segment (start 116.586 77.47) (end 118.872 79.756) (width 0.25) (layer F.Cu) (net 10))
 (segment (start 116.586 75.946) (end 116.586 77.47) (width 0.25) (layer F.Cu) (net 10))
 (segment (start 116.586 69.2785) (end 116.586 75.946) (width 0.25) (layer B.Cu) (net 10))
 (segment (start 117.9195 67.945) (end 116.586 69.2785) (width 0.25) (layer B.Cu) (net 10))
 (segment (start 124.9045 67.945) (end 117.9195 67.945) (width 0.25) (layer B.Cu) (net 10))
 (segment (start 130.3655 73.406) (end 124.9045 67.945) (width 0.25) (layer B.Cu) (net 10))
 (segment (start 140.5255 73.406) (end 130.3655 73.406) (width 0.25) (layer B.Cu) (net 10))
 (segment (start 146.780501 79.850999) (end 140.367001 79.850999) (width 0.25) (layer B.Cu) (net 12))
 (segment (start 149.724 76.9075) (end 146.780501 79.850999) (width 0.25) (layer B.Cu) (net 12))
 (segment (start 149.724 75.2475) (end 149.724 76.9075) (width 0.25) (layer B.Cu) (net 12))
 (segment (start 140.367001 79.850999) (end 137.795 82.423) (width 0.25) (layer B.Cu) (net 12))
 (segment (start 137.795 82.423) (end 137.795 82.423) (width 0.25) (layer B.Cu) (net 12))
 (via (at 137.795 82.423) (size 0.8) (drill 0.4) (layers F.Cu B.Cu) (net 12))
 (segment (start 136.668 83.55) (end 137.795 82.423) (width 0.25) (layer F.Cu) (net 12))
 (segment (start 136.668 84.6455) (end 136.668 83.55) (width 0.25) (layer F.Cu) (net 12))
 (segment (start 121.9835 86.106) (end 123.5075 86.106) (width 0.25) (layer F.Cu) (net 3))
 (segment (start 121.4755 85.598) (end 121.9835 86.106) (width 0.25) (layer F.Cu) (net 3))
 (segment (start 118.872 73.3265) (end 119.9355 73.3265) (width 0.25) (layer F.Cu) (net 3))
 (segment (start 121.4755 74.8665) (end 121.4755 85.598) (width 0.25) (layer F.Cu) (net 3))
 (segment (start 119.9355 73.3265) (end 121.4755 74.8665) (width 0.25) (layer F.Cu) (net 3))
 (segment (start 125.1585 88.646) (end 123.5075 88.646) (width 0.25) (layer B.Cu) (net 4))
 (segment (start 126.0475 87.757) (end 125.1585 88.646) (width 0.25) (layer B.Cu) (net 4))
 (segment (start 126.0475 71.12) (end 126.0475 87.757) (width 0.25) (layer B.Cu) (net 4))
 (segment (start 121.7295 74.422) (end 121.7295 70.993) (width 0.25) (layer B.Cu) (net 4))
 (segment (start 121.7295 70.993) (end 121.95175 70.77075) (width 0.25) (layer B.Cu) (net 4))
 (segment (start 121.95175 70.77075) (end 125.69825 70.77075) (width 0.25) (layer B.Cu) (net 4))
 (segment (start 125.69825 70.77075) (end 126.0475 71.12) (width 0.25) (layer B.Cu) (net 4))
 (segment (start 120.825 75.3265) (end 120.93575 75.21575) (width 0.25) (layer B.Cu) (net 4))
 (segment (start 118.872 75.3265) (end 120.825 75.3265) (width 0.25) (layer B.Cu) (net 4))
 (segment (start 120.93575 75.21575) (end 121.7295 74.422) (width 0.25) (layer B.Cu) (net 4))
 (segment (start 137.414 91.186) (end 146.431 91.186) (width 0.25) (layer B.Cu) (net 6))
 (segment (start 132.4365 96.1635) (end 137.414 91.186) (width 0.25) (layer B.Cu) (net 6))
 (segment (start 132.4365 96.1635) (end 119.947 96.1635) (width 0.25) (layer B.Cu) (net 6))
 (segment (start 133.2775 93.1635) (end 136.525 89.916) (width 0.25) (layer B.Cu) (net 7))
 (segment (start 145.161 89.916) (end 146.431 88.646) (width 0.25) (layer B.Cu) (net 7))
 (segment (start 136.525 89.916) (end 145.161 89.916) (width 0.25) (layer B.Cu) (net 7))
 (segment (start 133.2775 93.1635) (end 119.947 93.1635) (width 0.25) (layer B.Cu) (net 7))
 (segment (start 131.786 99.1635) (end 138.2395 92.71) (width 0.25) (layer B.Cu) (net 5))
 (segment (start 138.2395 92.71) (end 147.3835 92.71) (width 0.25) (layer B.Cu) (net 5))
 (segment (start 147.3835 92.71) (end 148.1455 91.948) (width 0.25) (layer B.Cu) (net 5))
 (segment (start 148.1455 91.948) (end 148.1455 85.852) (width 0.25) (layer B.Cu) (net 5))
 (segment (start 146.685 85.852) (end 146.431 86.106) (width 0.25) (layer B.Cu) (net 5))
 (segment (start 148.1455 85.852) (end 146.685 85.852) (width 0.25) (layer B.Cu) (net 5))
 (segment (start 131.786 99.1635) (end 119.947 99.1635) (width 0.25) (layer B.Cu) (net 5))
 (segment (start 146.431 81.026) (end 148.463 83.058) (width 0.25) (layer F.Cu) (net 18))
 (segment (start 148.463 83.5025) (end 151.384 86.4235) (width 0.25) (layer F.Cu) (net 18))
 (segment (start 148.463 83.058) (end 148.463 83.5025) (width 0.25) (layer F.Cu) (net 18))
 (segment (start 139.766 78.1255) (end 139.766 81.5696) (width 0.254) (layer F.Cu) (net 20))
 (segment (start 138.668 82.6676) (end 138.668 84.6455) (width 0.254) (layer F.Cu) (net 20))
 (segment (start 139.766 81.5696) (end 138.668 82.6676) (width 0.254) (layer F.Cu) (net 20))
 (segment (start 139.766 75.9255) (end 137.8712 77.8203) (width 0.254) (layer F.Cu) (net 21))
 (segment (start 137.8712 77.8203) (end 137.8712 81.1276) (width 0.254) (layer F.Cu) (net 21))
 (segment (start 137.8712 81.1276) (end 135.4836 83.5152) (width 0.254) (layer F.Cu) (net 21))
 (segment (start 135.4836 86.8901) (end 136.541 87.9475) (width 0.254) (layer F.Cu) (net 21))
 (segment (start 135.4836 83.5152) (end 135.4836 86.8901) (width 0.254) (layer F.Cu) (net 21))
 (segment (start 122.682 81.026) (end 123.5075 81.026) (width 0.25) (layer B.Cu) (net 8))
 (segment (start 118.872 84.836) (end 122.682 81.026) (width 0.25) (layer B.Cu) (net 8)))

